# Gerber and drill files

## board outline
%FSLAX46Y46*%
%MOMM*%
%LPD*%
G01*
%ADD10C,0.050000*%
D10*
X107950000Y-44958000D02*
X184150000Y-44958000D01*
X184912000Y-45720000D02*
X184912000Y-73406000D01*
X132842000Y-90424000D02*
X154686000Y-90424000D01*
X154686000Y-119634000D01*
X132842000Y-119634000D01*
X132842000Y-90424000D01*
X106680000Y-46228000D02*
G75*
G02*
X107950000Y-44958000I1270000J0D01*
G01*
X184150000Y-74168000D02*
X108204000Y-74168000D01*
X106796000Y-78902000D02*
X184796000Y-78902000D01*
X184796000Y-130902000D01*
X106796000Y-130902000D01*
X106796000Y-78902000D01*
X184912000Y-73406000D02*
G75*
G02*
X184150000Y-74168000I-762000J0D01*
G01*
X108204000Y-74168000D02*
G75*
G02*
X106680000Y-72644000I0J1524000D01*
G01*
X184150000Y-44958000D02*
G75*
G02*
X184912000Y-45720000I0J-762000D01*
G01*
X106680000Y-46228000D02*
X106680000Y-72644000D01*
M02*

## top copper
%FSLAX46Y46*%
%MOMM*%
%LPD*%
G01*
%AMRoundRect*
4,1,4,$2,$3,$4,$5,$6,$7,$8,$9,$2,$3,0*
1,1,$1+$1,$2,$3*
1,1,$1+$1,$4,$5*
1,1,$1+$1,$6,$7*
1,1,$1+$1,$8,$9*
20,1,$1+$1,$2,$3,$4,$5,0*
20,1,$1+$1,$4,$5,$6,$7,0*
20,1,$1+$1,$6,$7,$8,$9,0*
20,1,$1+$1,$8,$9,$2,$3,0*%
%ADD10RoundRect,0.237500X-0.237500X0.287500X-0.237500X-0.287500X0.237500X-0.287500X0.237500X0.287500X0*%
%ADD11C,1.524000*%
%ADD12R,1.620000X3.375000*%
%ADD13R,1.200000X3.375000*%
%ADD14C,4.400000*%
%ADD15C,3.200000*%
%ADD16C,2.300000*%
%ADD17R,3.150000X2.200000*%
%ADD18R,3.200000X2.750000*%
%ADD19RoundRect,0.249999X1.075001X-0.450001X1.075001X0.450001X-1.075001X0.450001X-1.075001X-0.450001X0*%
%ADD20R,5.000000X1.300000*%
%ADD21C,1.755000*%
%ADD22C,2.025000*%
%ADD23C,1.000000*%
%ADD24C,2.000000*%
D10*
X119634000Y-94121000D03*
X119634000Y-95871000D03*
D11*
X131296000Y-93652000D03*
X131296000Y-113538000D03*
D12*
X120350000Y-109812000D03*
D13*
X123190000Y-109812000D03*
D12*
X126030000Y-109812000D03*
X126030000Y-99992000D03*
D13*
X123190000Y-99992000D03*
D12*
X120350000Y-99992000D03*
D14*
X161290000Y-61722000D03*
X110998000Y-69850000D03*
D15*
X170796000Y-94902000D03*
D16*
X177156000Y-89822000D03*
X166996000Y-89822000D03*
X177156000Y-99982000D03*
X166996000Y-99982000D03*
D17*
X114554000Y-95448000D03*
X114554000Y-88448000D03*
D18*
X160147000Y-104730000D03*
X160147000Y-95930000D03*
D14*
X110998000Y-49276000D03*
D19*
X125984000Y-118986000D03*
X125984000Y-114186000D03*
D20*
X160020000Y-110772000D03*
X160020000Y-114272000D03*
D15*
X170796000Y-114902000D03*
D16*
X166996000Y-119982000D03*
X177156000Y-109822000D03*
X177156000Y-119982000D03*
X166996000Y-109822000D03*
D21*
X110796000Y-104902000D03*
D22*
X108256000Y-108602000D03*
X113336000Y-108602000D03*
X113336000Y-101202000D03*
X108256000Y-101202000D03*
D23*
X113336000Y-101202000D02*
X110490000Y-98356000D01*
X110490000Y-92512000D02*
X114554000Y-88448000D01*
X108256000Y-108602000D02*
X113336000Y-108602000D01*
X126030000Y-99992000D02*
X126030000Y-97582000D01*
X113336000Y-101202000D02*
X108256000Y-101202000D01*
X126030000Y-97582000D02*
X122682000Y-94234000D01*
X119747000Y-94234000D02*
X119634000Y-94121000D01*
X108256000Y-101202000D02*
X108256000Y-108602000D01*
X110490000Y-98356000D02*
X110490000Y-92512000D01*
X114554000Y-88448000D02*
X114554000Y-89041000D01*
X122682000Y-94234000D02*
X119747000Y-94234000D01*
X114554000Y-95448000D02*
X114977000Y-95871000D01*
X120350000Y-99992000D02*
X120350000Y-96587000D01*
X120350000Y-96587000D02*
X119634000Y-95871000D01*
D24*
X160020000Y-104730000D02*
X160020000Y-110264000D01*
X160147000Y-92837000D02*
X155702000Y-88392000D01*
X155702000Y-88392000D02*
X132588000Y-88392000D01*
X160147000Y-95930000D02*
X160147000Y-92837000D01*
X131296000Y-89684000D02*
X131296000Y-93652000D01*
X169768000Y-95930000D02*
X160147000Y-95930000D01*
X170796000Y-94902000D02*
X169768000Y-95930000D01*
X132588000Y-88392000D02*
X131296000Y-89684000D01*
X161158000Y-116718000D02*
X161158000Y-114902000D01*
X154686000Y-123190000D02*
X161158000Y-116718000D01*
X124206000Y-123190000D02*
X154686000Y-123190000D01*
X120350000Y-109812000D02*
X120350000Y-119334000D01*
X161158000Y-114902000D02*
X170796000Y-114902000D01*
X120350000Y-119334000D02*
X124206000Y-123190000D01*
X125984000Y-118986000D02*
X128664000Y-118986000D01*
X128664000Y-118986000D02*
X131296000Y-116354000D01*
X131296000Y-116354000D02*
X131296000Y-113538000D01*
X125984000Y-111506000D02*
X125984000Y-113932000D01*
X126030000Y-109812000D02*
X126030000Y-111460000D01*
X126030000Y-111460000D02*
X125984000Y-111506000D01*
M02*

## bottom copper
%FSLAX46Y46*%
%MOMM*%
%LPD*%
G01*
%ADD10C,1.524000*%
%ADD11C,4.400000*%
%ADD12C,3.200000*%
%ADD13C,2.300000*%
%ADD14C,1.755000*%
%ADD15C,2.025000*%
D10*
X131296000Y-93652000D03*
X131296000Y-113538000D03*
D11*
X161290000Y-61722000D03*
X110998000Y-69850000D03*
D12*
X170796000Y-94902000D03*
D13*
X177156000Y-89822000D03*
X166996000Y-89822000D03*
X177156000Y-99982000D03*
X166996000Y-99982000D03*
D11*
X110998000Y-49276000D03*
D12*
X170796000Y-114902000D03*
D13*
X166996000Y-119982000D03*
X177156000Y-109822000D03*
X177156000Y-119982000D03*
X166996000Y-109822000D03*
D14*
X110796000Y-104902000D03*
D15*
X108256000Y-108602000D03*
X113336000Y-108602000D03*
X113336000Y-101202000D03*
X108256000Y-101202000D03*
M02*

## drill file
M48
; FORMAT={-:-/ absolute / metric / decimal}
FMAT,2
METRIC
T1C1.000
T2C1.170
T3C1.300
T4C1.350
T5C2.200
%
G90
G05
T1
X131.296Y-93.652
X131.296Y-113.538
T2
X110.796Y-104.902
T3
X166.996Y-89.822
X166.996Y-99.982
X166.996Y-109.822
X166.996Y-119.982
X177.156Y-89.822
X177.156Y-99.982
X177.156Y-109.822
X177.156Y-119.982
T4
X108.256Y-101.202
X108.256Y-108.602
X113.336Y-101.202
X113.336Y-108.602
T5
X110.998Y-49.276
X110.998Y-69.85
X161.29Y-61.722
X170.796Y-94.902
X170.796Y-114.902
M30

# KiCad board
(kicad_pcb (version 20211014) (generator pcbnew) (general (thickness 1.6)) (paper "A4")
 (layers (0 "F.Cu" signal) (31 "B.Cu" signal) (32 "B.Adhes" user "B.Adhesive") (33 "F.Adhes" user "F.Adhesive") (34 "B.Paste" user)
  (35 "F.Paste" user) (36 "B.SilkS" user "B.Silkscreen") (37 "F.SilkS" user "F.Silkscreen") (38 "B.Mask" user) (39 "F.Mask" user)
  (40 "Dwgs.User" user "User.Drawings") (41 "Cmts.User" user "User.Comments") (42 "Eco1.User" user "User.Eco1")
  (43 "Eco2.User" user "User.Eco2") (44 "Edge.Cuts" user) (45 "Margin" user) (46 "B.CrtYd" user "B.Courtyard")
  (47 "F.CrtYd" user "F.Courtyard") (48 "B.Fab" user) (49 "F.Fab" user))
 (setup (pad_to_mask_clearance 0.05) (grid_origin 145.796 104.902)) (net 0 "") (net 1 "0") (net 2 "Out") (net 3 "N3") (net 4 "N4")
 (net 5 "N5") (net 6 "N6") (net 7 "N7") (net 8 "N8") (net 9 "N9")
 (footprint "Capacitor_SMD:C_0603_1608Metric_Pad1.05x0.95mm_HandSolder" (layer "F.Cu") (at 119.634 94.996 -90)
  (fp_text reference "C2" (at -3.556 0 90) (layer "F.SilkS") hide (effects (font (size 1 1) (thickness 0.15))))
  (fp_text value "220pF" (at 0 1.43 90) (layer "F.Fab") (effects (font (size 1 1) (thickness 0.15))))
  (pad "1" smd roundrect locked (at -0.875 0 270) (size 1.05 0.95) (layers "F.Cu" "F.Paste" "F.Mask") (roundrect_rratio 0.25) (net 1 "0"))
  (pad "2" smd roundrect locked (at 0.875 0 270) (size 1.05 0.95) (layers "F.Cu" "F.Paste" "F.Mask") (roundrect_rratio 0.25) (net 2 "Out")))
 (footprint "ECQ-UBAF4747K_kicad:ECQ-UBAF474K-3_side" (layer "F.Cu") (at 133.296 104.902 180)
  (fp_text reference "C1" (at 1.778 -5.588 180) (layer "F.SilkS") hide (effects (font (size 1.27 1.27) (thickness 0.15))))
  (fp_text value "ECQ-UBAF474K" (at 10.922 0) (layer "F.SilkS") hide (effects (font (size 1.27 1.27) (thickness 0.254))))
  (pad "1" thru_hole circle (at 2 11.25 180) (size 1.524 1.524) (drill 1) (layers *.Cu *.Mask) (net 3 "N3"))
  (pad "2" thru_hole circle (at 2 -8.636 180) (size 1.524 1.524) (drill 1) (layers *.Cu *.Mask) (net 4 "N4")))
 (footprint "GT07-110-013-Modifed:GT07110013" (layer "F.Cu") (at 123.19 104.902 180)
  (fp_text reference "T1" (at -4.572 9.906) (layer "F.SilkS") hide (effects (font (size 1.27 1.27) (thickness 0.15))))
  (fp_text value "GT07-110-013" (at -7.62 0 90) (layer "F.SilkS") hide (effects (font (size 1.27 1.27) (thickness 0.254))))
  (pad "1" smd rect (at 2.84 -4.91 180) (size 1.62 3.375) (layers "F.Cu" "F.Paste" "F.Mask") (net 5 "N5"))
  (pad "2" smd rect (at 0 -4.91 180) (size 1.2 3.375) (layers "F.Cu" "F.Paste" "F.Mask") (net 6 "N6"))
  (pad "3" smd rect (at -2.84 -4.91 180) (size 1.62 3.375) (layers "F.Cu" "F.Paste" "F.Mask") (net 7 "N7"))
  (pad "4" smd rect (at -2.84 4.91 180) (size 1.62 3.375) (layers "F.Cu" "F.Paste" "F.Mask") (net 1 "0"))
  (pad "5" smd rect (at 0 4.91 180) (size 1.2 3.375) (layers "F.Cu" "F.Paste" "F.Mask") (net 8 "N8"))
  (pad "6" smd rect (at 2.84 4.91 180) (size 1.62 3.375) (layers "F.Cu" "F.Paste" "F.Mask") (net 2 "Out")))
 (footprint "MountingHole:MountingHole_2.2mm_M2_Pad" (layer "F.Cu") (at 161.29 61.722)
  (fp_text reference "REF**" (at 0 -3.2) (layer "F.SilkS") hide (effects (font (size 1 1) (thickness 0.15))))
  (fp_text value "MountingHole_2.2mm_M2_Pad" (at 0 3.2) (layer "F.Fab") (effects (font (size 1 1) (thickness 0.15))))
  (pad "1" thru_hole circle locked (at 0 0) (size 4.4 4.4) (drill 2.2) (layers *.Cu *.Mask)))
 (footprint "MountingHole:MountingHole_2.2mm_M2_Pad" (layer "F.Cu") (at 110.998 69.85)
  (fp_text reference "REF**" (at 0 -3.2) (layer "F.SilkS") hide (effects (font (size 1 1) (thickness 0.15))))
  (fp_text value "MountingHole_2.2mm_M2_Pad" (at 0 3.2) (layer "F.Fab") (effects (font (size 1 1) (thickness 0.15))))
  (pad "1" thru_hole circle locked (at 0 0) (size 4.4 4.4) (drill 2.2) (layers *.Cu *.Mask)))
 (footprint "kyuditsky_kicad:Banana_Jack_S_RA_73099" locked (layer "F.Cu") (at 170.796 94.902)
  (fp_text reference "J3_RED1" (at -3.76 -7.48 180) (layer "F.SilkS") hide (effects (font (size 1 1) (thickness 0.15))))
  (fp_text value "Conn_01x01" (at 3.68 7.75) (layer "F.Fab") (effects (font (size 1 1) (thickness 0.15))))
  (pad "1" thru_hole circle locked (at 0 0) (size 3.2 3.2) (drill 2.2) (layers *.Cu *.Mask) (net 3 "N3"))
  (pad "2" thru_hole circle locked (at 6.36 -5.08) (size 2.3 2.3) (drill 1.3) (layers *.Cu *.Mask))
  (pad "2" thru_hole circle locked (at -3.8 -5.08) (size 2.3 2.3) (drill 1.3) (layers *.Cu *.Mask))
  (pad "2" thru_hole circle locked (at 6.36 5.08) (size 2.3 2.3) (drill 1.3) (layers *.Cu *.Mask))
  (pad "2" thru_hole circle locked (at -3.8 5.08) (size 2.3 2.3) (drill 1.3) (layers *.Cu *.Mask)))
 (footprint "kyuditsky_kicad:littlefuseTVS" (layer "F.Cu") (at 114.554 91.948 90)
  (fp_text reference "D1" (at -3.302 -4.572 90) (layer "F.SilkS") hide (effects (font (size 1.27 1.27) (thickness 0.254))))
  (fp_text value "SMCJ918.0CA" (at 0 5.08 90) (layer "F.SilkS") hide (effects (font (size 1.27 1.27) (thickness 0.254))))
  (pad "1" smd rect locked (at -3.5 0 90) (size 2.2 3.15) (layers "F.Cu" "F.Paste" "F.Mask") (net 2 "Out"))
  (pad "2" smd rect locked (at 3.5 0 90) (size 2.2 3.15) (layers "F.Cu" "F.Paste" "F.Mask") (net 1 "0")))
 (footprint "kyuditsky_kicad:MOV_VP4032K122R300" (layer "F.Cu") (at 160.02 100.33 90)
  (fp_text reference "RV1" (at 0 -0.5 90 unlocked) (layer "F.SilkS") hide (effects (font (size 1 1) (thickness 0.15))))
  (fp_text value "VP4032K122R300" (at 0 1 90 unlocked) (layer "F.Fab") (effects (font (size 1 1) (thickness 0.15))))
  (pad "1" smd rect (at -4.4 0.127 90) (size 2.75 3.2) (layers "F.Cu" "F.Paste" "F.Mask") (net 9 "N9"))
  (pad "2" smd rect (at 4.4 0.127 90) (size 2.75 3.2) (layers "F.Cu" "F.Paste" "F.Mask") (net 3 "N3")))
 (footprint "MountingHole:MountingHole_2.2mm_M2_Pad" (layer "F.Cu") (at 110.998 49.276)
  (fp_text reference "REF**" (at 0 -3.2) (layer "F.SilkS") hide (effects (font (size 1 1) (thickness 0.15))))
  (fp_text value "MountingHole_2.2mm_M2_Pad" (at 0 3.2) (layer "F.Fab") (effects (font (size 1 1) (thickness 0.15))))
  (pad "1" thru_hole circle locked (at 0 0) (size 4.4 4.4) (drill 2.2) (layers *.Cu *.Mask)))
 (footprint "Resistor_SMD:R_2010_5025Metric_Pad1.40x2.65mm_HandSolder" (layer "F.Cu") (at 125.984 116.586 90)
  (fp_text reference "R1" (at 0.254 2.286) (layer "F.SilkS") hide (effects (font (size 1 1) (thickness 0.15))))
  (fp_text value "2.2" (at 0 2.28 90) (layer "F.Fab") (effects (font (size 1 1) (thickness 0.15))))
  (pad "1" smd roundrect (at -2.4 0 90) (size 1.4 2.65) (layers "F.Cu" "F.Paste" "F.Mask") (roundrect_rratio 0.178571) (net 4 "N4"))
  (pad "2" smd roundrect (at 2.4 0 90) (size 1.4 2.65) (layers "F.Cu" "F.Paste" "F.Mask") (roundrect_rratio 0.178571) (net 7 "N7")))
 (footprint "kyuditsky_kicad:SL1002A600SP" (layer "F.Cu") (at 160.02 112.522 -90)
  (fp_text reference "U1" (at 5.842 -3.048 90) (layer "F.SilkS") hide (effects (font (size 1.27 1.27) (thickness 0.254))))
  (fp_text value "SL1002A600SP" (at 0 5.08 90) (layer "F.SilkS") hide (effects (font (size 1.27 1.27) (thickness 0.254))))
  (pad "1" smd rect locked (at -1.75 0 270) (size 1.3 5) (layers "F.Cu" "F.Paste" "F.Mask") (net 9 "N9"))
  (pad "2" smd rect locked (at 1.75 0 270) (size 1.3 5) (layers "F.Cu" "F.Paste" "F.Mask") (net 5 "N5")))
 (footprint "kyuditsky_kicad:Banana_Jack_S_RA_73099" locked (layer "F.Cu") (at 170.796 114.902)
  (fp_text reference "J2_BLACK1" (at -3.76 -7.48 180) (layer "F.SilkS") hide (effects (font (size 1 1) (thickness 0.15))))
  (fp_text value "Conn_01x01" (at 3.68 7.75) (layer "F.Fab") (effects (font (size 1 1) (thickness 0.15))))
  (pad "1" thru_hole circle locked (at 0 0) (size 3.2 3.2) (drill 2.2) (layers *.Cu *.Mask) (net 5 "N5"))
  (pad "2" thru_hole circle locked (at -3.8 5.08) (size 2.3 2.3) (drill 1.3) (layers *.Cu *.Mask))
  (pad "2" thru_hole circle locked (at 6.36 -5.08) (size 2.3 2.3) (drill 1.3) (layers *.Cu *.Mask))
  (pad "2" thru_hole circle locked (at 6.36 5.08) (size 2.3 2.3) (drill 1.3) (layers *.Cu *.Mask))
  (pad "2" thru_hole circle locked (at -3.8 -5.08) (size 2.3 2.3) (drill 1.3) (layers *.Cu *.Mask)))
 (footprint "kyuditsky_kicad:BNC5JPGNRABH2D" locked (layer "F.Cu") (at 110.796 104.902 90)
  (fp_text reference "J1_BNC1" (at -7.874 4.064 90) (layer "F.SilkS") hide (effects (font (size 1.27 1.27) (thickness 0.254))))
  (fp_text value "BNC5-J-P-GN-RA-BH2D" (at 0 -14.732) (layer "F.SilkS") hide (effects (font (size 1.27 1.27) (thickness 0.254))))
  (pad "1" thru_hole circle locked (at 0 0 90) (size 1.755 1.755) (drill 1.17) (layers *.Cu *.Mask) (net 2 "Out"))
  (pad "2" thru_hole circle locked (at -3.7 -2.54 90) (size 2.025 2.025) (drill 1.35) (layers *.Cu *.Mask) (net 1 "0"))
  (pad "3" thru_hole circle locked (at -3.7 2.54 90) (size 2.025 2.025) (drill 1.35) (layers *.Cu *.Mask) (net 1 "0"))
  (pad "4" thru_hole circle locked (at 3.7 2.54 90) (size 2.025 2.025) (drill 1.35) (layers *.Cu *.Mask) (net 1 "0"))
  (pad "5" thru_hole circle locked (at 3.7 -2.54 90) (size 2.025 2.025) (drill 1.35) (layers *.Cu *.Mask) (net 1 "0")))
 (gr_line (start 107.95 44.958) (end 184.15 44.958) (layer "Edge.Cuts") (width 0.05))
 (gr_line (start 184.912 45.72) (end 184.912 73.406) (layer "Edge.Cuts") (width 0.05))
 (gr_rect (start 132.842 90.424) (end 154.686 119.634) (layer "Edge.Cuts") (width 0.05) (fill none))
 (gr_arc (start 106.68 46.228) (mid 107.051974 45.329974) (end 107.95 44.958) (layer "Edge.Cuts") (width 0.05))
 (gr_line (start 184.15 74.168) (end 108.204 74.168) (layer "Edge.Cuts") (width 0.05))
 (gr_rect locked (start 106.796 78.902) (end 184.796 130.902) (layer "Edge.Cuts") (width 0.05) (fill none))
 (gr_arc (start 184.912 73.406) (mid 184.688815 73.944815) (end 184.15 74.168) (layer "Edge.Cuts") (width 0.05))
 (gr_arc (start 108.204 74.168) (mid 107.126369 73.721631) (end 106.68 72.644) (layer "Edge.Cuts") (width 0.05))
 (gr_arc (start 184.15 44.958) (mid 184.688815 45.181185) (end 184.912 45.72) (layer "Edge.Cuts") (width 0.05))
 (gr_line (start 106.68 46.228) (end 106.68 72.644) (layer "Edge.Cuts") (width 0.05))
 (segment (start 113.336 101.202) (end 110.49 98.356) (width 1) (layer "F.Cu") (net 1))
 (segment (start 110.49 92.512) (end 114.554 88.448) (width 1) (layer "F.Cu") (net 1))
 (segment (start 108.256 108.602) (end 113.336 108.602) (width 1) (layer "F.Cu") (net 1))
 (segment (start 126.03 99.992) (end 126.03 97.582) (width 1) (layer "F.Cu") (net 1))
 (segment (start 113.336 101.202) (end 108.256 101.202) (width 1) (layer "F.Cu") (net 1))
 (segment (start 126.03 97.582) (end 122.682 94.234) (width 1) (layer "F.Cu") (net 1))
 (segment (start 119.747 94.234) (end 119.634 94.121) (width 1) (layer "F.Cu") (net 1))
 (segment (start 108.256 101.202) (end 108.256 108.602) (width 1) (layer "F.Cu") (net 1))
 (segment (start 110.49 98.356) (end 110.49 92.512) (width 1) (layer "F.Cu") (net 1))
 (segment (start 114.554 88.448) (end 114.554 89.041) (width 1) (layer "F.Cu") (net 1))
 (segment (start 122.682 94.234) (end 119.747 94.234) (width 1) (layer "F.Cu") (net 1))
 (segment (start 114.554 95.448) (end 114.977 95.871) (width 1) (layer "F.Cu") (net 2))
 (segment (start 120.35 99.992) (end 120.35 96.587) (width 1) (layer "F.Cu") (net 2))
 (segment (start 120.35 96.587) (end 119.634 95.871) (width 1) (layer "F.Cu") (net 2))
 (segment (start 160.02 104.73) (end 160.02 110.264) (width 2) (layer "F.Cu") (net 9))
 (segment (start 160.147 92.837) (end 155.702 88.392) (width 2) (layer "F.Cu") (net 3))
 (segment (start 155.702 88.392) (end 132.588 88.392) (width 2) (layer "F.Cu") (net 3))
 (segment (start 160.147 95.93) (end 160.147 92.837) (width 2) (layer "F.Cu") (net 3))
 (segment (start 131.296 89.684) (end 131.296 93.652) (width 2) (layer "F.Cu") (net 3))
 (segment (start 169.768 95.93) (end 160.147 95.93) (width 2) (layer "F.Cu") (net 3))
 (segment (start 170.796 94.902) (end 169.768 95.93) (width 2) (layer "F.Cu") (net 3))
 (segment (start 132.588 88.392) (end 131.296 89.684) (width 2) (layer "F.Cu") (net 3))
 (segment (start 161.158 116.718) (end 161.158 114.902) (width 2) (layer "F.Cu") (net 5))
 (segment (start 154.686 123.19) (end 161.158 116.718) (width 2) (layer "F.Cu") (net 5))
 (segment (start 124.206 123.19) (end 154.686 123.19) (width 2) (layer "F.Cu") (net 5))
 (segment (start 120.35 109.812) (end 120.35 119.334) (width 2) (layer "F.Cu") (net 5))
 (segment (start 161.158 114.902) (end 170.796 114.902) (width 2) (layer "F.Cu") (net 5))
 (segment (start 120.35 119.334) (end 124.206 123.19) (width 2) (layer "F.Cu") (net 5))
 (segment (start 125.984 118.986) (end 128.664 118.986) (width 2) (layer "F.Cu") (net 4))
 (segment (start 128.664 118.986) (end 131.296 116.354) (width 2) (layer "F.Cu") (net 4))
 (segment (start 131.296 116.354) (end 131.296 113.538) (width 2) (layer "F.Cu") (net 4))
 (segment (start 125.984 111.506) (end 125.984 113.932) (width 2) (layer "F.Cu") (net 7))
 (segment (start 126.03 109.812) (end 126.03 111.46) (width 2) (layer "F.Cu") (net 7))
 (segment (start 126.03 111.46) (end 125.984 111.506) (width 2) (layer "F.Cu") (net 7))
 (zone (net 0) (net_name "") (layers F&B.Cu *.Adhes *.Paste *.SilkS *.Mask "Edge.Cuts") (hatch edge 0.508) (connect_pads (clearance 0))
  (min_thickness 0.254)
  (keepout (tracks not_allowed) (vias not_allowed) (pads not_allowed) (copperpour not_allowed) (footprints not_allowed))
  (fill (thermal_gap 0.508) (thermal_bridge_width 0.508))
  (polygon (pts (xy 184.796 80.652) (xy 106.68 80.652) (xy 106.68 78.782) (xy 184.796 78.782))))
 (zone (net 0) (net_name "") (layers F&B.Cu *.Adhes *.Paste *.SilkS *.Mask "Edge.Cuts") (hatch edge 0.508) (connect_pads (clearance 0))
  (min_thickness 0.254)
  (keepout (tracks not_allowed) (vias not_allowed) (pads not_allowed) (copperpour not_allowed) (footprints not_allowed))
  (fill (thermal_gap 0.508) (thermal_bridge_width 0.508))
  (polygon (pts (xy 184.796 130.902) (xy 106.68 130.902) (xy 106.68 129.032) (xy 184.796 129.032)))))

